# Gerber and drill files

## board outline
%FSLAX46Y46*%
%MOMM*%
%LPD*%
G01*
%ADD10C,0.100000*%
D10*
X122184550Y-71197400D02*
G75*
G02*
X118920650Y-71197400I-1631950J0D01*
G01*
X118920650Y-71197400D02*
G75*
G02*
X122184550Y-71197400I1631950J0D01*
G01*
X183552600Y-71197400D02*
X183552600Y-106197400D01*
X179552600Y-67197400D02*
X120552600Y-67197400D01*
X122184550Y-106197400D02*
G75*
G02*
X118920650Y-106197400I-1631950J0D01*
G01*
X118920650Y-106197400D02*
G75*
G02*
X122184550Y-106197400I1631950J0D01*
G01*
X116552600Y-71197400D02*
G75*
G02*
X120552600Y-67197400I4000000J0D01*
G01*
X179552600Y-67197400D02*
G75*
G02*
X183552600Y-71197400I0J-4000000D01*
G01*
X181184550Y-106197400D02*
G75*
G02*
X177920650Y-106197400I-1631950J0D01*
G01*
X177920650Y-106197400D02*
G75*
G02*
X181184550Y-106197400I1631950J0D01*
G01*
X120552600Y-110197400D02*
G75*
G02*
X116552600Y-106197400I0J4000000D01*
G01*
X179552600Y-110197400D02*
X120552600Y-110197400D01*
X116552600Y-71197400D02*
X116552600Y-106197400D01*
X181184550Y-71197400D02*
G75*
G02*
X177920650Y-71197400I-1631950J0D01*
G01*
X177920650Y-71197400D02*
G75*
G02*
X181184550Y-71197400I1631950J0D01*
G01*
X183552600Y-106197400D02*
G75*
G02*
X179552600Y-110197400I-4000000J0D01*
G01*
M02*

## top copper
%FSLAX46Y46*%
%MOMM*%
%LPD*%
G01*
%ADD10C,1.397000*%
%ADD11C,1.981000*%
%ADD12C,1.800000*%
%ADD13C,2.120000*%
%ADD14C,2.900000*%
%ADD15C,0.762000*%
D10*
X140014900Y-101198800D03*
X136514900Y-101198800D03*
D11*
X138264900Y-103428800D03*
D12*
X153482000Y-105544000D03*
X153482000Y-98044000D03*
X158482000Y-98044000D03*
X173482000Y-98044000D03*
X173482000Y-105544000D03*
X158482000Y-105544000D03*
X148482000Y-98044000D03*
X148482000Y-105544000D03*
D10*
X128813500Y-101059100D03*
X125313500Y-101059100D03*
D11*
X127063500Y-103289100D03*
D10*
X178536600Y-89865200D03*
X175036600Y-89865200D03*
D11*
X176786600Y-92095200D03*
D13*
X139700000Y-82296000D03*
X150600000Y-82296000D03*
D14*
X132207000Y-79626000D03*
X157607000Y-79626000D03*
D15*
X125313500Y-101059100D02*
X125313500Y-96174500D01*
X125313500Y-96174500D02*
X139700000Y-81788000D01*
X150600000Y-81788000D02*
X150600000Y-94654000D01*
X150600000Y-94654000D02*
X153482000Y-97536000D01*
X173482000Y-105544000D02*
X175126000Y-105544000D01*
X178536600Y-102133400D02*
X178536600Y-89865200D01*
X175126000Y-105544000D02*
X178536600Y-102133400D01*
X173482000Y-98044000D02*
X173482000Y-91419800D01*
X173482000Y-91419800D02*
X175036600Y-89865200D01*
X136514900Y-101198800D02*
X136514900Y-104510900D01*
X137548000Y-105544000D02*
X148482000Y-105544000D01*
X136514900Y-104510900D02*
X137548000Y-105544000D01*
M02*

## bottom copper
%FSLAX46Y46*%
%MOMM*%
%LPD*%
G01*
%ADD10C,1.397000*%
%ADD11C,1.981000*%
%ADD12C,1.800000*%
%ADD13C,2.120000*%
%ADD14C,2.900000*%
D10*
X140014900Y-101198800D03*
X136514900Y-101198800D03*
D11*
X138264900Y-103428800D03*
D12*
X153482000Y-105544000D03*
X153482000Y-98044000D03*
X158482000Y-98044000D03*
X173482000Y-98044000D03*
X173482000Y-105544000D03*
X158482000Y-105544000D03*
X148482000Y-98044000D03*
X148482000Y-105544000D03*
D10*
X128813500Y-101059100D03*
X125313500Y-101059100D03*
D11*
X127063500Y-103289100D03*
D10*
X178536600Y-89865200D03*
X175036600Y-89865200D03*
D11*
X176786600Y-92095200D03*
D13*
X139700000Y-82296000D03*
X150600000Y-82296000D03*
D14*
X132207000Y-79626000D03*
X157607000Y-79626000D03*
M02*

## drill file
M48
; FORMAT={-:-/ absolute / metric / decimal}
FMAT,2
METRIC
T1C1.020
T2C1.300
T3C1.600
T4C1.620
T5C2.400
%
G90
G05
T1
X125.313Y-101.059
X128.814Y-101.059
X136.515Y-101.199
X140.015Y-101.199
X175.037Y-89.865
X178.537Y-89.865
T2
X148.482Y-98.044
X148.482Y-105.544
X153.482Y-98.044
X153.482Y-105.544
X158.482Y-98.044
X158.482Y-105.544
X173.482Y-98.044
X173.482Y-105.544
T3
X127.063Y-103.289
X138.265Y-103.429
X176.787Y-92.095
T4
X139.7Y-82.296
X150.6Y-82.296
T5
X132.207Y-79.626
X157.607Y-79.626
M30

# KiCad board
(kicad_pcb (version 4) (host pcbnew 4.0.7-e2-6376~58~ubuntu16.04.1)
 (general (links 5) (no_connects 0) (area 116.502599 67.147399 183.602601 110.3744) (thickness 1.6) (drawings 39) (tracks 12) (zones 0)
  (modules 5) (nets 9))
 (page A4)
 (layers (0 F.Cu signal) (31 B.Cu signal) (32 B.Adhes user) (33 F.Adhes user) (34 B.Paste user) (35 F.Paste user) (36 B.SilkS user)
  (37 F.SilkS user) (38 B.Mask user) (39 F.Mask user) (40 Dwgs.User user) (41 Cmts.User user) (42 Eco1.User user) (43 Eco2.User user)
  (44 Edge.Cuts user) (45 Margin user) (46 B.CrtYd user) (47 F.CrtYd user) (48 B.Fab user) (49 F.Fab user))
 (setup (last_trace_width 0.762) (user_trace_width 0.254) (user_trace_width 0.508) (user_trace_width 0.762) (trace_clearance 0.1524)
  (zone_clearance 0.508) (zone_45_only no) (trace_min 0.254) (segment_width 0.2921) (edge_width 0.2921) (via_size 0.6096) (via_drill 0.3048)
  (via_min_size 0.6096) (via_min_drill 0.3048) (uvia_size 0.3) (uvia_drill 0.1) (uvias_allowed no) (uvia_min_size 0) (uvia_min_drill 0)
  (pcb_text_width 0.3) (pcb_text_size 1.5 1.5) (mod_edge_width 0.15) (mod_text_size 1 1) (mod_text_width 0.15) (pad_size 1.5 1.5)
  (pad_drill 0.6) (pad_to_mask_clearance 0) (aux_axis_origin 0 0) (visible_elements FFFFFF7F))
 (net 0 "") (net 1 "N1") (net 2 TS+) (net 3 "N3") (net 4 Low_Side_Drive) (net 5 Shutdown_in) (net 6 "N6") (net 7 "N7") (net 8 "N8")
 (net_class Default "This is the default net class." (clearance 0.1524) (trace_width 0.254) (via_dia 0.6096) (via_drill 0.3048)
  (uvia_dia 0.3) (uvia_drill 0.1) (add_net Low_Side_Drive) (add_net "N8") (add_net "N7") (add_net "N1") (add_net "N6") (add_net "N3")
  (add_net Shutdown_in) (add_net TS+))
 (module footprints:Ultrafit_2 (layer F.Cu) (at 140.0149 101.1988 270)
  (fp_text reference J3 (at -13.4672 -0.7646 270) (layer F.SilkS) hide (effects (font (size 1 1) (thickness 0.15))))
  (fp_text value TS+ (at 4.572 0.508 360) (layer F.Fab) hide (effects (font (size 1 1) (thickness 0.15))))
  (pad 2 thru_hole circle (at 0 0 270) (size 1.397 1.397) (drill 1.02) (layers *.Cu *.Mask) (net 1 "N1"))
  (pad 1 thru_hole circle (at 0 3.5 270) (size 1.397 1.397) (drill 1.02) (layers *.Cu *.Mask) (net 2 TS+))
  (pad "" thru_hole circle (at 2.23 1.75 270) (size 1.981 1.981) (drill 1.6) (layers *.Cu *.Mask)))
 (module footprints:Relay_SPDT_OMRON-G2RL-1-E (layer F.Cu) (at 173.482 98.044 180)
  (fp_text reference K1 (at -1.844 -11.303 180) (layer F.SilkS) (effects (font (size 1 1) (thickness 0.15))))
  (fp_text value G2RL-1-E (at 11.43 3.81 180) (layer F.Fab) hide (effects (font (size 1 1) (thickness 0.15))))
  (pad 3 thru_hole circle (at 20 -7.5 180) (size 1.8 1.8) (drill 1.3) (layers *.Cu *.Mask))
  (pad 6 thru_hole circle (at 20 0 180) (size 1.8 1.8) (drill 1.3) (layers *.Cu *.Mask) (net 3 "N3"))
  (pad 7 thru_hole circle (at 15 0 180) (size 1.8 1.8) (drill 1.3) (layers *.Cu *.Mask))
  (pad 8 thru_hole circle (at 0 0 180) (size 1.8 1.8) (drill 1.3) (layers *.Cu *.Mask) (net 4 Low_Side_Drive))
  (pad 1 thru_hole circle (at 0 -7.5 180) (size 1.8 1.8) (drill 1.3) (layers *.Cu *.Mask) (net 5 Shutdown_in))
  (pad 2 thru_hole circle (at 15 -7.5 180) (size 1.8 1.8) (drill 1.3) (layers *.Cu *.Mask) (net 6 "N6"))
  (pad 5 thru_hole circle (at 25 0 180) (size 1.8 1.8) (drill 1.3) (layers *.Cu *.Mask))
  (pad 4 thru_hole circle (at 25 -7.5 180) (size 1.8 1.8) (drill 1.3) (layers *.Cu *.Mask) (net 2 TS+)))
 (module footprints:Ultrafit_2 (layer F.Cu) (at 128.8135 101.0591 270)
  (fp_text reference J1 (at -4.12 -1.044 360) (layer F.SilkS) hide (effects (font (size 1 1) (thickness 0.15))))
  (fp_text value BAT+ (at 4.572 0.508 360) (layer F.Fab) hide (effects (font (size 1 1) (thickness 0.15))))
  (pad 2 thru_hole circle (at 0 0 270) (size 1.397 1.397) (drill 1.02) (layers *.Cu *.Mask) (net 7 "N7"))
  (pad 1 thru_hole circle (at 0 3.5 270) (size 1.397 1.397) (drill 1.02) (layers *.Cu *.Mask) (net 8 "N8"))
  (pad "" thru_hole circle (at 2.23 1.75 270) (size 1.981 1.981) (drill 1.6) (layers *.Cu *.Mask)))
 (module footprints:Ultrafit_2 (layer F.Cu) (at 178.5366 89.8652 270)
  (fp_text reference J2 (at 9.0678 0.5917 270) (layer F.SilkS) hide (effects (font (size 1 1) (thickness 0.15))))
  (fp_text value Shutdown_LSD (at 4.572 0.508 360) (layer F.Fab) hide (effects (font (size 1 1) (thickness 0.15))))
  (pad 2 thru_hole circle (at 0 0 270) (size 1.397 1.397) (drill 1.02) (layers *.Cu *.Mask) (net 5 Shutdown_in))
  (pad 1 thru_hole circle (at 0 3.5 270) (size 1.397 1.397) (drill 1.02) (layers *.Cu *.Mask) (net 4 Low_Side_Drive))
  (pad "" thru_hole circle (at 2.23 1.75 270) (size 1.981 1.981) (drill 1.6) (layers *.Cu *.Mask)))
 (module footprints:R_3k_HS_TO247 (layer F.Cu) (at 139.7 82.296)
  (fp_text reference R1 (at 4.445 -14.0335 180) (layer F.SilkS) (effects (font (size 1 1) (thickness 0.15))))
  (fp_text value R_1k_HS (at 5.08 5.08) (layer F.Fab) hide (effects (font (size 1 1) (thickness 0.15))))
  (pad 1 thru_hole circle (at 0 0) (size 2.12 2.12) (drill 1.62) (layers *.Cu *.Mask) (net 8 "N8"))
  (pad 2 thru_hole circle (at 10.9 0) (size 2.12 2.12) (drill 1.62) (layers *.Cu *.Mask) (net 3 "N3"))
  (pad 4 thru_hole circle (at -7.493 -2.67) (size 2.9 2.9) (drill 2.4) (layers *.Cu *.Mask))
  (pad 5 thru_hole circle (at 17.907 -2.67) (size 2.9 2.9) (drill 2.4) (layers *.Cu *.Mask)))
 (gr_circle (center 120.5526 71.1974) (end 122.18455 71.1974) (layer Edge.Cuts) (width 0.1))
 (gr_line (start 183.5526 71.1974) (end 183.5526 106.1974) (layer Edge.Cuts) (width 0.1))
 (gr_line (start 179.5526 67.1974) (end 120.5526 67.1974) (layer Edge.Cuts) (width 0.1))
 (gr_circle (center 120.5526 106.1974) (end 122.18455 106.1974) (layer Edge.Cuts) (width 0.1))
 (gr_arc (start 120.5526 71.1974) (end 120.5526 67.1974) (angle -90) (layer Edge.Cuts) (width 0.1))
 (gr_arc (start 179.5526 71.1974) (end 183.5526 71.1974) (angle -90) (layer Edge.Cuts) (width 0.1))
 (gr_circle (center 179.5526 106.1974) (end 181.18455 106.1974) (layer Edge.Cuts) (width 0.1))
 (gr_arc (start 120.5526 106.1974) (end 116.5526 106.1974) (angle -90) (layer Edge.Cuts) (width 0.1))
 (gr_line (start 179.5526 110.1974) (end 120.5526 110.1974) (layer Edge.Cuts) (width 0.1))
 (gr_line (start 116.5526 71.1974) (end 116.5526 106.1974) (layer Edge.Cuts) (width 0.1))
 (gr_circle (center 179.5526 71.1974) (end 181.18455 71.1974) (layer Edge.Cuts) (width 0.1))
 (gr_arc (start 179.5526 106.1974) (end 179.5526 110.1974) (angle -90) (layer Edge.Cuts) (width 0.1))
 (segment (start 125.3135 101.0591) (end 125.3135 96.1745) (width 0.762) (layer F.Cu) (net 8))
 (segment (start 125.3135 96.1745) (end 139.7 81.788) (width 0.762) (layer F.Cu) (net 8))
 (segment (start 150.6 81.788) (end 150.6 94.654) (width 0.762) (layer F.Cu) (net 3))
 (segment (start 150.6 94.654) (end 153.482 97.536) (width 0.762) (layer F.Cu) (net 3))
 (segment (start 173.482 105.544) (end 175.126 105.544) (width 0.762) (layer F.Cu) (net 5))
 (segment (start 178.5366 102.1334) (end 178.5366 89.8652) (width 0.762) (layer F.Cu) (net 5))
 (segment (start 175.126 105.544) (end 178.5366 102.1334) (width 0.762) (layer F.Cu) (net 5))
 (segment (start 173.482 98.044) (end 173.482 91.4198) (width 0.762) (layer F.Cu) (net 4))
 (segment (start 173.482 91.4198) (end 175.0366 89.8652) (width 0.762) (layer F.Cu) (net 4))
 (segment (start 136.5149 101.1988) (end 136.5149 104.5109) (width 0.762) (layer F.Cu) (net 2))
 (segment (start 137.548 105.544) (end 148.482 105.544) (width 0.762) (layer F.Cu) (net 2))
 (segment (start 136.5149 104.5109) (end 137.548 105.544) (width 0.762) (layer F.Cu) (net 2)))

